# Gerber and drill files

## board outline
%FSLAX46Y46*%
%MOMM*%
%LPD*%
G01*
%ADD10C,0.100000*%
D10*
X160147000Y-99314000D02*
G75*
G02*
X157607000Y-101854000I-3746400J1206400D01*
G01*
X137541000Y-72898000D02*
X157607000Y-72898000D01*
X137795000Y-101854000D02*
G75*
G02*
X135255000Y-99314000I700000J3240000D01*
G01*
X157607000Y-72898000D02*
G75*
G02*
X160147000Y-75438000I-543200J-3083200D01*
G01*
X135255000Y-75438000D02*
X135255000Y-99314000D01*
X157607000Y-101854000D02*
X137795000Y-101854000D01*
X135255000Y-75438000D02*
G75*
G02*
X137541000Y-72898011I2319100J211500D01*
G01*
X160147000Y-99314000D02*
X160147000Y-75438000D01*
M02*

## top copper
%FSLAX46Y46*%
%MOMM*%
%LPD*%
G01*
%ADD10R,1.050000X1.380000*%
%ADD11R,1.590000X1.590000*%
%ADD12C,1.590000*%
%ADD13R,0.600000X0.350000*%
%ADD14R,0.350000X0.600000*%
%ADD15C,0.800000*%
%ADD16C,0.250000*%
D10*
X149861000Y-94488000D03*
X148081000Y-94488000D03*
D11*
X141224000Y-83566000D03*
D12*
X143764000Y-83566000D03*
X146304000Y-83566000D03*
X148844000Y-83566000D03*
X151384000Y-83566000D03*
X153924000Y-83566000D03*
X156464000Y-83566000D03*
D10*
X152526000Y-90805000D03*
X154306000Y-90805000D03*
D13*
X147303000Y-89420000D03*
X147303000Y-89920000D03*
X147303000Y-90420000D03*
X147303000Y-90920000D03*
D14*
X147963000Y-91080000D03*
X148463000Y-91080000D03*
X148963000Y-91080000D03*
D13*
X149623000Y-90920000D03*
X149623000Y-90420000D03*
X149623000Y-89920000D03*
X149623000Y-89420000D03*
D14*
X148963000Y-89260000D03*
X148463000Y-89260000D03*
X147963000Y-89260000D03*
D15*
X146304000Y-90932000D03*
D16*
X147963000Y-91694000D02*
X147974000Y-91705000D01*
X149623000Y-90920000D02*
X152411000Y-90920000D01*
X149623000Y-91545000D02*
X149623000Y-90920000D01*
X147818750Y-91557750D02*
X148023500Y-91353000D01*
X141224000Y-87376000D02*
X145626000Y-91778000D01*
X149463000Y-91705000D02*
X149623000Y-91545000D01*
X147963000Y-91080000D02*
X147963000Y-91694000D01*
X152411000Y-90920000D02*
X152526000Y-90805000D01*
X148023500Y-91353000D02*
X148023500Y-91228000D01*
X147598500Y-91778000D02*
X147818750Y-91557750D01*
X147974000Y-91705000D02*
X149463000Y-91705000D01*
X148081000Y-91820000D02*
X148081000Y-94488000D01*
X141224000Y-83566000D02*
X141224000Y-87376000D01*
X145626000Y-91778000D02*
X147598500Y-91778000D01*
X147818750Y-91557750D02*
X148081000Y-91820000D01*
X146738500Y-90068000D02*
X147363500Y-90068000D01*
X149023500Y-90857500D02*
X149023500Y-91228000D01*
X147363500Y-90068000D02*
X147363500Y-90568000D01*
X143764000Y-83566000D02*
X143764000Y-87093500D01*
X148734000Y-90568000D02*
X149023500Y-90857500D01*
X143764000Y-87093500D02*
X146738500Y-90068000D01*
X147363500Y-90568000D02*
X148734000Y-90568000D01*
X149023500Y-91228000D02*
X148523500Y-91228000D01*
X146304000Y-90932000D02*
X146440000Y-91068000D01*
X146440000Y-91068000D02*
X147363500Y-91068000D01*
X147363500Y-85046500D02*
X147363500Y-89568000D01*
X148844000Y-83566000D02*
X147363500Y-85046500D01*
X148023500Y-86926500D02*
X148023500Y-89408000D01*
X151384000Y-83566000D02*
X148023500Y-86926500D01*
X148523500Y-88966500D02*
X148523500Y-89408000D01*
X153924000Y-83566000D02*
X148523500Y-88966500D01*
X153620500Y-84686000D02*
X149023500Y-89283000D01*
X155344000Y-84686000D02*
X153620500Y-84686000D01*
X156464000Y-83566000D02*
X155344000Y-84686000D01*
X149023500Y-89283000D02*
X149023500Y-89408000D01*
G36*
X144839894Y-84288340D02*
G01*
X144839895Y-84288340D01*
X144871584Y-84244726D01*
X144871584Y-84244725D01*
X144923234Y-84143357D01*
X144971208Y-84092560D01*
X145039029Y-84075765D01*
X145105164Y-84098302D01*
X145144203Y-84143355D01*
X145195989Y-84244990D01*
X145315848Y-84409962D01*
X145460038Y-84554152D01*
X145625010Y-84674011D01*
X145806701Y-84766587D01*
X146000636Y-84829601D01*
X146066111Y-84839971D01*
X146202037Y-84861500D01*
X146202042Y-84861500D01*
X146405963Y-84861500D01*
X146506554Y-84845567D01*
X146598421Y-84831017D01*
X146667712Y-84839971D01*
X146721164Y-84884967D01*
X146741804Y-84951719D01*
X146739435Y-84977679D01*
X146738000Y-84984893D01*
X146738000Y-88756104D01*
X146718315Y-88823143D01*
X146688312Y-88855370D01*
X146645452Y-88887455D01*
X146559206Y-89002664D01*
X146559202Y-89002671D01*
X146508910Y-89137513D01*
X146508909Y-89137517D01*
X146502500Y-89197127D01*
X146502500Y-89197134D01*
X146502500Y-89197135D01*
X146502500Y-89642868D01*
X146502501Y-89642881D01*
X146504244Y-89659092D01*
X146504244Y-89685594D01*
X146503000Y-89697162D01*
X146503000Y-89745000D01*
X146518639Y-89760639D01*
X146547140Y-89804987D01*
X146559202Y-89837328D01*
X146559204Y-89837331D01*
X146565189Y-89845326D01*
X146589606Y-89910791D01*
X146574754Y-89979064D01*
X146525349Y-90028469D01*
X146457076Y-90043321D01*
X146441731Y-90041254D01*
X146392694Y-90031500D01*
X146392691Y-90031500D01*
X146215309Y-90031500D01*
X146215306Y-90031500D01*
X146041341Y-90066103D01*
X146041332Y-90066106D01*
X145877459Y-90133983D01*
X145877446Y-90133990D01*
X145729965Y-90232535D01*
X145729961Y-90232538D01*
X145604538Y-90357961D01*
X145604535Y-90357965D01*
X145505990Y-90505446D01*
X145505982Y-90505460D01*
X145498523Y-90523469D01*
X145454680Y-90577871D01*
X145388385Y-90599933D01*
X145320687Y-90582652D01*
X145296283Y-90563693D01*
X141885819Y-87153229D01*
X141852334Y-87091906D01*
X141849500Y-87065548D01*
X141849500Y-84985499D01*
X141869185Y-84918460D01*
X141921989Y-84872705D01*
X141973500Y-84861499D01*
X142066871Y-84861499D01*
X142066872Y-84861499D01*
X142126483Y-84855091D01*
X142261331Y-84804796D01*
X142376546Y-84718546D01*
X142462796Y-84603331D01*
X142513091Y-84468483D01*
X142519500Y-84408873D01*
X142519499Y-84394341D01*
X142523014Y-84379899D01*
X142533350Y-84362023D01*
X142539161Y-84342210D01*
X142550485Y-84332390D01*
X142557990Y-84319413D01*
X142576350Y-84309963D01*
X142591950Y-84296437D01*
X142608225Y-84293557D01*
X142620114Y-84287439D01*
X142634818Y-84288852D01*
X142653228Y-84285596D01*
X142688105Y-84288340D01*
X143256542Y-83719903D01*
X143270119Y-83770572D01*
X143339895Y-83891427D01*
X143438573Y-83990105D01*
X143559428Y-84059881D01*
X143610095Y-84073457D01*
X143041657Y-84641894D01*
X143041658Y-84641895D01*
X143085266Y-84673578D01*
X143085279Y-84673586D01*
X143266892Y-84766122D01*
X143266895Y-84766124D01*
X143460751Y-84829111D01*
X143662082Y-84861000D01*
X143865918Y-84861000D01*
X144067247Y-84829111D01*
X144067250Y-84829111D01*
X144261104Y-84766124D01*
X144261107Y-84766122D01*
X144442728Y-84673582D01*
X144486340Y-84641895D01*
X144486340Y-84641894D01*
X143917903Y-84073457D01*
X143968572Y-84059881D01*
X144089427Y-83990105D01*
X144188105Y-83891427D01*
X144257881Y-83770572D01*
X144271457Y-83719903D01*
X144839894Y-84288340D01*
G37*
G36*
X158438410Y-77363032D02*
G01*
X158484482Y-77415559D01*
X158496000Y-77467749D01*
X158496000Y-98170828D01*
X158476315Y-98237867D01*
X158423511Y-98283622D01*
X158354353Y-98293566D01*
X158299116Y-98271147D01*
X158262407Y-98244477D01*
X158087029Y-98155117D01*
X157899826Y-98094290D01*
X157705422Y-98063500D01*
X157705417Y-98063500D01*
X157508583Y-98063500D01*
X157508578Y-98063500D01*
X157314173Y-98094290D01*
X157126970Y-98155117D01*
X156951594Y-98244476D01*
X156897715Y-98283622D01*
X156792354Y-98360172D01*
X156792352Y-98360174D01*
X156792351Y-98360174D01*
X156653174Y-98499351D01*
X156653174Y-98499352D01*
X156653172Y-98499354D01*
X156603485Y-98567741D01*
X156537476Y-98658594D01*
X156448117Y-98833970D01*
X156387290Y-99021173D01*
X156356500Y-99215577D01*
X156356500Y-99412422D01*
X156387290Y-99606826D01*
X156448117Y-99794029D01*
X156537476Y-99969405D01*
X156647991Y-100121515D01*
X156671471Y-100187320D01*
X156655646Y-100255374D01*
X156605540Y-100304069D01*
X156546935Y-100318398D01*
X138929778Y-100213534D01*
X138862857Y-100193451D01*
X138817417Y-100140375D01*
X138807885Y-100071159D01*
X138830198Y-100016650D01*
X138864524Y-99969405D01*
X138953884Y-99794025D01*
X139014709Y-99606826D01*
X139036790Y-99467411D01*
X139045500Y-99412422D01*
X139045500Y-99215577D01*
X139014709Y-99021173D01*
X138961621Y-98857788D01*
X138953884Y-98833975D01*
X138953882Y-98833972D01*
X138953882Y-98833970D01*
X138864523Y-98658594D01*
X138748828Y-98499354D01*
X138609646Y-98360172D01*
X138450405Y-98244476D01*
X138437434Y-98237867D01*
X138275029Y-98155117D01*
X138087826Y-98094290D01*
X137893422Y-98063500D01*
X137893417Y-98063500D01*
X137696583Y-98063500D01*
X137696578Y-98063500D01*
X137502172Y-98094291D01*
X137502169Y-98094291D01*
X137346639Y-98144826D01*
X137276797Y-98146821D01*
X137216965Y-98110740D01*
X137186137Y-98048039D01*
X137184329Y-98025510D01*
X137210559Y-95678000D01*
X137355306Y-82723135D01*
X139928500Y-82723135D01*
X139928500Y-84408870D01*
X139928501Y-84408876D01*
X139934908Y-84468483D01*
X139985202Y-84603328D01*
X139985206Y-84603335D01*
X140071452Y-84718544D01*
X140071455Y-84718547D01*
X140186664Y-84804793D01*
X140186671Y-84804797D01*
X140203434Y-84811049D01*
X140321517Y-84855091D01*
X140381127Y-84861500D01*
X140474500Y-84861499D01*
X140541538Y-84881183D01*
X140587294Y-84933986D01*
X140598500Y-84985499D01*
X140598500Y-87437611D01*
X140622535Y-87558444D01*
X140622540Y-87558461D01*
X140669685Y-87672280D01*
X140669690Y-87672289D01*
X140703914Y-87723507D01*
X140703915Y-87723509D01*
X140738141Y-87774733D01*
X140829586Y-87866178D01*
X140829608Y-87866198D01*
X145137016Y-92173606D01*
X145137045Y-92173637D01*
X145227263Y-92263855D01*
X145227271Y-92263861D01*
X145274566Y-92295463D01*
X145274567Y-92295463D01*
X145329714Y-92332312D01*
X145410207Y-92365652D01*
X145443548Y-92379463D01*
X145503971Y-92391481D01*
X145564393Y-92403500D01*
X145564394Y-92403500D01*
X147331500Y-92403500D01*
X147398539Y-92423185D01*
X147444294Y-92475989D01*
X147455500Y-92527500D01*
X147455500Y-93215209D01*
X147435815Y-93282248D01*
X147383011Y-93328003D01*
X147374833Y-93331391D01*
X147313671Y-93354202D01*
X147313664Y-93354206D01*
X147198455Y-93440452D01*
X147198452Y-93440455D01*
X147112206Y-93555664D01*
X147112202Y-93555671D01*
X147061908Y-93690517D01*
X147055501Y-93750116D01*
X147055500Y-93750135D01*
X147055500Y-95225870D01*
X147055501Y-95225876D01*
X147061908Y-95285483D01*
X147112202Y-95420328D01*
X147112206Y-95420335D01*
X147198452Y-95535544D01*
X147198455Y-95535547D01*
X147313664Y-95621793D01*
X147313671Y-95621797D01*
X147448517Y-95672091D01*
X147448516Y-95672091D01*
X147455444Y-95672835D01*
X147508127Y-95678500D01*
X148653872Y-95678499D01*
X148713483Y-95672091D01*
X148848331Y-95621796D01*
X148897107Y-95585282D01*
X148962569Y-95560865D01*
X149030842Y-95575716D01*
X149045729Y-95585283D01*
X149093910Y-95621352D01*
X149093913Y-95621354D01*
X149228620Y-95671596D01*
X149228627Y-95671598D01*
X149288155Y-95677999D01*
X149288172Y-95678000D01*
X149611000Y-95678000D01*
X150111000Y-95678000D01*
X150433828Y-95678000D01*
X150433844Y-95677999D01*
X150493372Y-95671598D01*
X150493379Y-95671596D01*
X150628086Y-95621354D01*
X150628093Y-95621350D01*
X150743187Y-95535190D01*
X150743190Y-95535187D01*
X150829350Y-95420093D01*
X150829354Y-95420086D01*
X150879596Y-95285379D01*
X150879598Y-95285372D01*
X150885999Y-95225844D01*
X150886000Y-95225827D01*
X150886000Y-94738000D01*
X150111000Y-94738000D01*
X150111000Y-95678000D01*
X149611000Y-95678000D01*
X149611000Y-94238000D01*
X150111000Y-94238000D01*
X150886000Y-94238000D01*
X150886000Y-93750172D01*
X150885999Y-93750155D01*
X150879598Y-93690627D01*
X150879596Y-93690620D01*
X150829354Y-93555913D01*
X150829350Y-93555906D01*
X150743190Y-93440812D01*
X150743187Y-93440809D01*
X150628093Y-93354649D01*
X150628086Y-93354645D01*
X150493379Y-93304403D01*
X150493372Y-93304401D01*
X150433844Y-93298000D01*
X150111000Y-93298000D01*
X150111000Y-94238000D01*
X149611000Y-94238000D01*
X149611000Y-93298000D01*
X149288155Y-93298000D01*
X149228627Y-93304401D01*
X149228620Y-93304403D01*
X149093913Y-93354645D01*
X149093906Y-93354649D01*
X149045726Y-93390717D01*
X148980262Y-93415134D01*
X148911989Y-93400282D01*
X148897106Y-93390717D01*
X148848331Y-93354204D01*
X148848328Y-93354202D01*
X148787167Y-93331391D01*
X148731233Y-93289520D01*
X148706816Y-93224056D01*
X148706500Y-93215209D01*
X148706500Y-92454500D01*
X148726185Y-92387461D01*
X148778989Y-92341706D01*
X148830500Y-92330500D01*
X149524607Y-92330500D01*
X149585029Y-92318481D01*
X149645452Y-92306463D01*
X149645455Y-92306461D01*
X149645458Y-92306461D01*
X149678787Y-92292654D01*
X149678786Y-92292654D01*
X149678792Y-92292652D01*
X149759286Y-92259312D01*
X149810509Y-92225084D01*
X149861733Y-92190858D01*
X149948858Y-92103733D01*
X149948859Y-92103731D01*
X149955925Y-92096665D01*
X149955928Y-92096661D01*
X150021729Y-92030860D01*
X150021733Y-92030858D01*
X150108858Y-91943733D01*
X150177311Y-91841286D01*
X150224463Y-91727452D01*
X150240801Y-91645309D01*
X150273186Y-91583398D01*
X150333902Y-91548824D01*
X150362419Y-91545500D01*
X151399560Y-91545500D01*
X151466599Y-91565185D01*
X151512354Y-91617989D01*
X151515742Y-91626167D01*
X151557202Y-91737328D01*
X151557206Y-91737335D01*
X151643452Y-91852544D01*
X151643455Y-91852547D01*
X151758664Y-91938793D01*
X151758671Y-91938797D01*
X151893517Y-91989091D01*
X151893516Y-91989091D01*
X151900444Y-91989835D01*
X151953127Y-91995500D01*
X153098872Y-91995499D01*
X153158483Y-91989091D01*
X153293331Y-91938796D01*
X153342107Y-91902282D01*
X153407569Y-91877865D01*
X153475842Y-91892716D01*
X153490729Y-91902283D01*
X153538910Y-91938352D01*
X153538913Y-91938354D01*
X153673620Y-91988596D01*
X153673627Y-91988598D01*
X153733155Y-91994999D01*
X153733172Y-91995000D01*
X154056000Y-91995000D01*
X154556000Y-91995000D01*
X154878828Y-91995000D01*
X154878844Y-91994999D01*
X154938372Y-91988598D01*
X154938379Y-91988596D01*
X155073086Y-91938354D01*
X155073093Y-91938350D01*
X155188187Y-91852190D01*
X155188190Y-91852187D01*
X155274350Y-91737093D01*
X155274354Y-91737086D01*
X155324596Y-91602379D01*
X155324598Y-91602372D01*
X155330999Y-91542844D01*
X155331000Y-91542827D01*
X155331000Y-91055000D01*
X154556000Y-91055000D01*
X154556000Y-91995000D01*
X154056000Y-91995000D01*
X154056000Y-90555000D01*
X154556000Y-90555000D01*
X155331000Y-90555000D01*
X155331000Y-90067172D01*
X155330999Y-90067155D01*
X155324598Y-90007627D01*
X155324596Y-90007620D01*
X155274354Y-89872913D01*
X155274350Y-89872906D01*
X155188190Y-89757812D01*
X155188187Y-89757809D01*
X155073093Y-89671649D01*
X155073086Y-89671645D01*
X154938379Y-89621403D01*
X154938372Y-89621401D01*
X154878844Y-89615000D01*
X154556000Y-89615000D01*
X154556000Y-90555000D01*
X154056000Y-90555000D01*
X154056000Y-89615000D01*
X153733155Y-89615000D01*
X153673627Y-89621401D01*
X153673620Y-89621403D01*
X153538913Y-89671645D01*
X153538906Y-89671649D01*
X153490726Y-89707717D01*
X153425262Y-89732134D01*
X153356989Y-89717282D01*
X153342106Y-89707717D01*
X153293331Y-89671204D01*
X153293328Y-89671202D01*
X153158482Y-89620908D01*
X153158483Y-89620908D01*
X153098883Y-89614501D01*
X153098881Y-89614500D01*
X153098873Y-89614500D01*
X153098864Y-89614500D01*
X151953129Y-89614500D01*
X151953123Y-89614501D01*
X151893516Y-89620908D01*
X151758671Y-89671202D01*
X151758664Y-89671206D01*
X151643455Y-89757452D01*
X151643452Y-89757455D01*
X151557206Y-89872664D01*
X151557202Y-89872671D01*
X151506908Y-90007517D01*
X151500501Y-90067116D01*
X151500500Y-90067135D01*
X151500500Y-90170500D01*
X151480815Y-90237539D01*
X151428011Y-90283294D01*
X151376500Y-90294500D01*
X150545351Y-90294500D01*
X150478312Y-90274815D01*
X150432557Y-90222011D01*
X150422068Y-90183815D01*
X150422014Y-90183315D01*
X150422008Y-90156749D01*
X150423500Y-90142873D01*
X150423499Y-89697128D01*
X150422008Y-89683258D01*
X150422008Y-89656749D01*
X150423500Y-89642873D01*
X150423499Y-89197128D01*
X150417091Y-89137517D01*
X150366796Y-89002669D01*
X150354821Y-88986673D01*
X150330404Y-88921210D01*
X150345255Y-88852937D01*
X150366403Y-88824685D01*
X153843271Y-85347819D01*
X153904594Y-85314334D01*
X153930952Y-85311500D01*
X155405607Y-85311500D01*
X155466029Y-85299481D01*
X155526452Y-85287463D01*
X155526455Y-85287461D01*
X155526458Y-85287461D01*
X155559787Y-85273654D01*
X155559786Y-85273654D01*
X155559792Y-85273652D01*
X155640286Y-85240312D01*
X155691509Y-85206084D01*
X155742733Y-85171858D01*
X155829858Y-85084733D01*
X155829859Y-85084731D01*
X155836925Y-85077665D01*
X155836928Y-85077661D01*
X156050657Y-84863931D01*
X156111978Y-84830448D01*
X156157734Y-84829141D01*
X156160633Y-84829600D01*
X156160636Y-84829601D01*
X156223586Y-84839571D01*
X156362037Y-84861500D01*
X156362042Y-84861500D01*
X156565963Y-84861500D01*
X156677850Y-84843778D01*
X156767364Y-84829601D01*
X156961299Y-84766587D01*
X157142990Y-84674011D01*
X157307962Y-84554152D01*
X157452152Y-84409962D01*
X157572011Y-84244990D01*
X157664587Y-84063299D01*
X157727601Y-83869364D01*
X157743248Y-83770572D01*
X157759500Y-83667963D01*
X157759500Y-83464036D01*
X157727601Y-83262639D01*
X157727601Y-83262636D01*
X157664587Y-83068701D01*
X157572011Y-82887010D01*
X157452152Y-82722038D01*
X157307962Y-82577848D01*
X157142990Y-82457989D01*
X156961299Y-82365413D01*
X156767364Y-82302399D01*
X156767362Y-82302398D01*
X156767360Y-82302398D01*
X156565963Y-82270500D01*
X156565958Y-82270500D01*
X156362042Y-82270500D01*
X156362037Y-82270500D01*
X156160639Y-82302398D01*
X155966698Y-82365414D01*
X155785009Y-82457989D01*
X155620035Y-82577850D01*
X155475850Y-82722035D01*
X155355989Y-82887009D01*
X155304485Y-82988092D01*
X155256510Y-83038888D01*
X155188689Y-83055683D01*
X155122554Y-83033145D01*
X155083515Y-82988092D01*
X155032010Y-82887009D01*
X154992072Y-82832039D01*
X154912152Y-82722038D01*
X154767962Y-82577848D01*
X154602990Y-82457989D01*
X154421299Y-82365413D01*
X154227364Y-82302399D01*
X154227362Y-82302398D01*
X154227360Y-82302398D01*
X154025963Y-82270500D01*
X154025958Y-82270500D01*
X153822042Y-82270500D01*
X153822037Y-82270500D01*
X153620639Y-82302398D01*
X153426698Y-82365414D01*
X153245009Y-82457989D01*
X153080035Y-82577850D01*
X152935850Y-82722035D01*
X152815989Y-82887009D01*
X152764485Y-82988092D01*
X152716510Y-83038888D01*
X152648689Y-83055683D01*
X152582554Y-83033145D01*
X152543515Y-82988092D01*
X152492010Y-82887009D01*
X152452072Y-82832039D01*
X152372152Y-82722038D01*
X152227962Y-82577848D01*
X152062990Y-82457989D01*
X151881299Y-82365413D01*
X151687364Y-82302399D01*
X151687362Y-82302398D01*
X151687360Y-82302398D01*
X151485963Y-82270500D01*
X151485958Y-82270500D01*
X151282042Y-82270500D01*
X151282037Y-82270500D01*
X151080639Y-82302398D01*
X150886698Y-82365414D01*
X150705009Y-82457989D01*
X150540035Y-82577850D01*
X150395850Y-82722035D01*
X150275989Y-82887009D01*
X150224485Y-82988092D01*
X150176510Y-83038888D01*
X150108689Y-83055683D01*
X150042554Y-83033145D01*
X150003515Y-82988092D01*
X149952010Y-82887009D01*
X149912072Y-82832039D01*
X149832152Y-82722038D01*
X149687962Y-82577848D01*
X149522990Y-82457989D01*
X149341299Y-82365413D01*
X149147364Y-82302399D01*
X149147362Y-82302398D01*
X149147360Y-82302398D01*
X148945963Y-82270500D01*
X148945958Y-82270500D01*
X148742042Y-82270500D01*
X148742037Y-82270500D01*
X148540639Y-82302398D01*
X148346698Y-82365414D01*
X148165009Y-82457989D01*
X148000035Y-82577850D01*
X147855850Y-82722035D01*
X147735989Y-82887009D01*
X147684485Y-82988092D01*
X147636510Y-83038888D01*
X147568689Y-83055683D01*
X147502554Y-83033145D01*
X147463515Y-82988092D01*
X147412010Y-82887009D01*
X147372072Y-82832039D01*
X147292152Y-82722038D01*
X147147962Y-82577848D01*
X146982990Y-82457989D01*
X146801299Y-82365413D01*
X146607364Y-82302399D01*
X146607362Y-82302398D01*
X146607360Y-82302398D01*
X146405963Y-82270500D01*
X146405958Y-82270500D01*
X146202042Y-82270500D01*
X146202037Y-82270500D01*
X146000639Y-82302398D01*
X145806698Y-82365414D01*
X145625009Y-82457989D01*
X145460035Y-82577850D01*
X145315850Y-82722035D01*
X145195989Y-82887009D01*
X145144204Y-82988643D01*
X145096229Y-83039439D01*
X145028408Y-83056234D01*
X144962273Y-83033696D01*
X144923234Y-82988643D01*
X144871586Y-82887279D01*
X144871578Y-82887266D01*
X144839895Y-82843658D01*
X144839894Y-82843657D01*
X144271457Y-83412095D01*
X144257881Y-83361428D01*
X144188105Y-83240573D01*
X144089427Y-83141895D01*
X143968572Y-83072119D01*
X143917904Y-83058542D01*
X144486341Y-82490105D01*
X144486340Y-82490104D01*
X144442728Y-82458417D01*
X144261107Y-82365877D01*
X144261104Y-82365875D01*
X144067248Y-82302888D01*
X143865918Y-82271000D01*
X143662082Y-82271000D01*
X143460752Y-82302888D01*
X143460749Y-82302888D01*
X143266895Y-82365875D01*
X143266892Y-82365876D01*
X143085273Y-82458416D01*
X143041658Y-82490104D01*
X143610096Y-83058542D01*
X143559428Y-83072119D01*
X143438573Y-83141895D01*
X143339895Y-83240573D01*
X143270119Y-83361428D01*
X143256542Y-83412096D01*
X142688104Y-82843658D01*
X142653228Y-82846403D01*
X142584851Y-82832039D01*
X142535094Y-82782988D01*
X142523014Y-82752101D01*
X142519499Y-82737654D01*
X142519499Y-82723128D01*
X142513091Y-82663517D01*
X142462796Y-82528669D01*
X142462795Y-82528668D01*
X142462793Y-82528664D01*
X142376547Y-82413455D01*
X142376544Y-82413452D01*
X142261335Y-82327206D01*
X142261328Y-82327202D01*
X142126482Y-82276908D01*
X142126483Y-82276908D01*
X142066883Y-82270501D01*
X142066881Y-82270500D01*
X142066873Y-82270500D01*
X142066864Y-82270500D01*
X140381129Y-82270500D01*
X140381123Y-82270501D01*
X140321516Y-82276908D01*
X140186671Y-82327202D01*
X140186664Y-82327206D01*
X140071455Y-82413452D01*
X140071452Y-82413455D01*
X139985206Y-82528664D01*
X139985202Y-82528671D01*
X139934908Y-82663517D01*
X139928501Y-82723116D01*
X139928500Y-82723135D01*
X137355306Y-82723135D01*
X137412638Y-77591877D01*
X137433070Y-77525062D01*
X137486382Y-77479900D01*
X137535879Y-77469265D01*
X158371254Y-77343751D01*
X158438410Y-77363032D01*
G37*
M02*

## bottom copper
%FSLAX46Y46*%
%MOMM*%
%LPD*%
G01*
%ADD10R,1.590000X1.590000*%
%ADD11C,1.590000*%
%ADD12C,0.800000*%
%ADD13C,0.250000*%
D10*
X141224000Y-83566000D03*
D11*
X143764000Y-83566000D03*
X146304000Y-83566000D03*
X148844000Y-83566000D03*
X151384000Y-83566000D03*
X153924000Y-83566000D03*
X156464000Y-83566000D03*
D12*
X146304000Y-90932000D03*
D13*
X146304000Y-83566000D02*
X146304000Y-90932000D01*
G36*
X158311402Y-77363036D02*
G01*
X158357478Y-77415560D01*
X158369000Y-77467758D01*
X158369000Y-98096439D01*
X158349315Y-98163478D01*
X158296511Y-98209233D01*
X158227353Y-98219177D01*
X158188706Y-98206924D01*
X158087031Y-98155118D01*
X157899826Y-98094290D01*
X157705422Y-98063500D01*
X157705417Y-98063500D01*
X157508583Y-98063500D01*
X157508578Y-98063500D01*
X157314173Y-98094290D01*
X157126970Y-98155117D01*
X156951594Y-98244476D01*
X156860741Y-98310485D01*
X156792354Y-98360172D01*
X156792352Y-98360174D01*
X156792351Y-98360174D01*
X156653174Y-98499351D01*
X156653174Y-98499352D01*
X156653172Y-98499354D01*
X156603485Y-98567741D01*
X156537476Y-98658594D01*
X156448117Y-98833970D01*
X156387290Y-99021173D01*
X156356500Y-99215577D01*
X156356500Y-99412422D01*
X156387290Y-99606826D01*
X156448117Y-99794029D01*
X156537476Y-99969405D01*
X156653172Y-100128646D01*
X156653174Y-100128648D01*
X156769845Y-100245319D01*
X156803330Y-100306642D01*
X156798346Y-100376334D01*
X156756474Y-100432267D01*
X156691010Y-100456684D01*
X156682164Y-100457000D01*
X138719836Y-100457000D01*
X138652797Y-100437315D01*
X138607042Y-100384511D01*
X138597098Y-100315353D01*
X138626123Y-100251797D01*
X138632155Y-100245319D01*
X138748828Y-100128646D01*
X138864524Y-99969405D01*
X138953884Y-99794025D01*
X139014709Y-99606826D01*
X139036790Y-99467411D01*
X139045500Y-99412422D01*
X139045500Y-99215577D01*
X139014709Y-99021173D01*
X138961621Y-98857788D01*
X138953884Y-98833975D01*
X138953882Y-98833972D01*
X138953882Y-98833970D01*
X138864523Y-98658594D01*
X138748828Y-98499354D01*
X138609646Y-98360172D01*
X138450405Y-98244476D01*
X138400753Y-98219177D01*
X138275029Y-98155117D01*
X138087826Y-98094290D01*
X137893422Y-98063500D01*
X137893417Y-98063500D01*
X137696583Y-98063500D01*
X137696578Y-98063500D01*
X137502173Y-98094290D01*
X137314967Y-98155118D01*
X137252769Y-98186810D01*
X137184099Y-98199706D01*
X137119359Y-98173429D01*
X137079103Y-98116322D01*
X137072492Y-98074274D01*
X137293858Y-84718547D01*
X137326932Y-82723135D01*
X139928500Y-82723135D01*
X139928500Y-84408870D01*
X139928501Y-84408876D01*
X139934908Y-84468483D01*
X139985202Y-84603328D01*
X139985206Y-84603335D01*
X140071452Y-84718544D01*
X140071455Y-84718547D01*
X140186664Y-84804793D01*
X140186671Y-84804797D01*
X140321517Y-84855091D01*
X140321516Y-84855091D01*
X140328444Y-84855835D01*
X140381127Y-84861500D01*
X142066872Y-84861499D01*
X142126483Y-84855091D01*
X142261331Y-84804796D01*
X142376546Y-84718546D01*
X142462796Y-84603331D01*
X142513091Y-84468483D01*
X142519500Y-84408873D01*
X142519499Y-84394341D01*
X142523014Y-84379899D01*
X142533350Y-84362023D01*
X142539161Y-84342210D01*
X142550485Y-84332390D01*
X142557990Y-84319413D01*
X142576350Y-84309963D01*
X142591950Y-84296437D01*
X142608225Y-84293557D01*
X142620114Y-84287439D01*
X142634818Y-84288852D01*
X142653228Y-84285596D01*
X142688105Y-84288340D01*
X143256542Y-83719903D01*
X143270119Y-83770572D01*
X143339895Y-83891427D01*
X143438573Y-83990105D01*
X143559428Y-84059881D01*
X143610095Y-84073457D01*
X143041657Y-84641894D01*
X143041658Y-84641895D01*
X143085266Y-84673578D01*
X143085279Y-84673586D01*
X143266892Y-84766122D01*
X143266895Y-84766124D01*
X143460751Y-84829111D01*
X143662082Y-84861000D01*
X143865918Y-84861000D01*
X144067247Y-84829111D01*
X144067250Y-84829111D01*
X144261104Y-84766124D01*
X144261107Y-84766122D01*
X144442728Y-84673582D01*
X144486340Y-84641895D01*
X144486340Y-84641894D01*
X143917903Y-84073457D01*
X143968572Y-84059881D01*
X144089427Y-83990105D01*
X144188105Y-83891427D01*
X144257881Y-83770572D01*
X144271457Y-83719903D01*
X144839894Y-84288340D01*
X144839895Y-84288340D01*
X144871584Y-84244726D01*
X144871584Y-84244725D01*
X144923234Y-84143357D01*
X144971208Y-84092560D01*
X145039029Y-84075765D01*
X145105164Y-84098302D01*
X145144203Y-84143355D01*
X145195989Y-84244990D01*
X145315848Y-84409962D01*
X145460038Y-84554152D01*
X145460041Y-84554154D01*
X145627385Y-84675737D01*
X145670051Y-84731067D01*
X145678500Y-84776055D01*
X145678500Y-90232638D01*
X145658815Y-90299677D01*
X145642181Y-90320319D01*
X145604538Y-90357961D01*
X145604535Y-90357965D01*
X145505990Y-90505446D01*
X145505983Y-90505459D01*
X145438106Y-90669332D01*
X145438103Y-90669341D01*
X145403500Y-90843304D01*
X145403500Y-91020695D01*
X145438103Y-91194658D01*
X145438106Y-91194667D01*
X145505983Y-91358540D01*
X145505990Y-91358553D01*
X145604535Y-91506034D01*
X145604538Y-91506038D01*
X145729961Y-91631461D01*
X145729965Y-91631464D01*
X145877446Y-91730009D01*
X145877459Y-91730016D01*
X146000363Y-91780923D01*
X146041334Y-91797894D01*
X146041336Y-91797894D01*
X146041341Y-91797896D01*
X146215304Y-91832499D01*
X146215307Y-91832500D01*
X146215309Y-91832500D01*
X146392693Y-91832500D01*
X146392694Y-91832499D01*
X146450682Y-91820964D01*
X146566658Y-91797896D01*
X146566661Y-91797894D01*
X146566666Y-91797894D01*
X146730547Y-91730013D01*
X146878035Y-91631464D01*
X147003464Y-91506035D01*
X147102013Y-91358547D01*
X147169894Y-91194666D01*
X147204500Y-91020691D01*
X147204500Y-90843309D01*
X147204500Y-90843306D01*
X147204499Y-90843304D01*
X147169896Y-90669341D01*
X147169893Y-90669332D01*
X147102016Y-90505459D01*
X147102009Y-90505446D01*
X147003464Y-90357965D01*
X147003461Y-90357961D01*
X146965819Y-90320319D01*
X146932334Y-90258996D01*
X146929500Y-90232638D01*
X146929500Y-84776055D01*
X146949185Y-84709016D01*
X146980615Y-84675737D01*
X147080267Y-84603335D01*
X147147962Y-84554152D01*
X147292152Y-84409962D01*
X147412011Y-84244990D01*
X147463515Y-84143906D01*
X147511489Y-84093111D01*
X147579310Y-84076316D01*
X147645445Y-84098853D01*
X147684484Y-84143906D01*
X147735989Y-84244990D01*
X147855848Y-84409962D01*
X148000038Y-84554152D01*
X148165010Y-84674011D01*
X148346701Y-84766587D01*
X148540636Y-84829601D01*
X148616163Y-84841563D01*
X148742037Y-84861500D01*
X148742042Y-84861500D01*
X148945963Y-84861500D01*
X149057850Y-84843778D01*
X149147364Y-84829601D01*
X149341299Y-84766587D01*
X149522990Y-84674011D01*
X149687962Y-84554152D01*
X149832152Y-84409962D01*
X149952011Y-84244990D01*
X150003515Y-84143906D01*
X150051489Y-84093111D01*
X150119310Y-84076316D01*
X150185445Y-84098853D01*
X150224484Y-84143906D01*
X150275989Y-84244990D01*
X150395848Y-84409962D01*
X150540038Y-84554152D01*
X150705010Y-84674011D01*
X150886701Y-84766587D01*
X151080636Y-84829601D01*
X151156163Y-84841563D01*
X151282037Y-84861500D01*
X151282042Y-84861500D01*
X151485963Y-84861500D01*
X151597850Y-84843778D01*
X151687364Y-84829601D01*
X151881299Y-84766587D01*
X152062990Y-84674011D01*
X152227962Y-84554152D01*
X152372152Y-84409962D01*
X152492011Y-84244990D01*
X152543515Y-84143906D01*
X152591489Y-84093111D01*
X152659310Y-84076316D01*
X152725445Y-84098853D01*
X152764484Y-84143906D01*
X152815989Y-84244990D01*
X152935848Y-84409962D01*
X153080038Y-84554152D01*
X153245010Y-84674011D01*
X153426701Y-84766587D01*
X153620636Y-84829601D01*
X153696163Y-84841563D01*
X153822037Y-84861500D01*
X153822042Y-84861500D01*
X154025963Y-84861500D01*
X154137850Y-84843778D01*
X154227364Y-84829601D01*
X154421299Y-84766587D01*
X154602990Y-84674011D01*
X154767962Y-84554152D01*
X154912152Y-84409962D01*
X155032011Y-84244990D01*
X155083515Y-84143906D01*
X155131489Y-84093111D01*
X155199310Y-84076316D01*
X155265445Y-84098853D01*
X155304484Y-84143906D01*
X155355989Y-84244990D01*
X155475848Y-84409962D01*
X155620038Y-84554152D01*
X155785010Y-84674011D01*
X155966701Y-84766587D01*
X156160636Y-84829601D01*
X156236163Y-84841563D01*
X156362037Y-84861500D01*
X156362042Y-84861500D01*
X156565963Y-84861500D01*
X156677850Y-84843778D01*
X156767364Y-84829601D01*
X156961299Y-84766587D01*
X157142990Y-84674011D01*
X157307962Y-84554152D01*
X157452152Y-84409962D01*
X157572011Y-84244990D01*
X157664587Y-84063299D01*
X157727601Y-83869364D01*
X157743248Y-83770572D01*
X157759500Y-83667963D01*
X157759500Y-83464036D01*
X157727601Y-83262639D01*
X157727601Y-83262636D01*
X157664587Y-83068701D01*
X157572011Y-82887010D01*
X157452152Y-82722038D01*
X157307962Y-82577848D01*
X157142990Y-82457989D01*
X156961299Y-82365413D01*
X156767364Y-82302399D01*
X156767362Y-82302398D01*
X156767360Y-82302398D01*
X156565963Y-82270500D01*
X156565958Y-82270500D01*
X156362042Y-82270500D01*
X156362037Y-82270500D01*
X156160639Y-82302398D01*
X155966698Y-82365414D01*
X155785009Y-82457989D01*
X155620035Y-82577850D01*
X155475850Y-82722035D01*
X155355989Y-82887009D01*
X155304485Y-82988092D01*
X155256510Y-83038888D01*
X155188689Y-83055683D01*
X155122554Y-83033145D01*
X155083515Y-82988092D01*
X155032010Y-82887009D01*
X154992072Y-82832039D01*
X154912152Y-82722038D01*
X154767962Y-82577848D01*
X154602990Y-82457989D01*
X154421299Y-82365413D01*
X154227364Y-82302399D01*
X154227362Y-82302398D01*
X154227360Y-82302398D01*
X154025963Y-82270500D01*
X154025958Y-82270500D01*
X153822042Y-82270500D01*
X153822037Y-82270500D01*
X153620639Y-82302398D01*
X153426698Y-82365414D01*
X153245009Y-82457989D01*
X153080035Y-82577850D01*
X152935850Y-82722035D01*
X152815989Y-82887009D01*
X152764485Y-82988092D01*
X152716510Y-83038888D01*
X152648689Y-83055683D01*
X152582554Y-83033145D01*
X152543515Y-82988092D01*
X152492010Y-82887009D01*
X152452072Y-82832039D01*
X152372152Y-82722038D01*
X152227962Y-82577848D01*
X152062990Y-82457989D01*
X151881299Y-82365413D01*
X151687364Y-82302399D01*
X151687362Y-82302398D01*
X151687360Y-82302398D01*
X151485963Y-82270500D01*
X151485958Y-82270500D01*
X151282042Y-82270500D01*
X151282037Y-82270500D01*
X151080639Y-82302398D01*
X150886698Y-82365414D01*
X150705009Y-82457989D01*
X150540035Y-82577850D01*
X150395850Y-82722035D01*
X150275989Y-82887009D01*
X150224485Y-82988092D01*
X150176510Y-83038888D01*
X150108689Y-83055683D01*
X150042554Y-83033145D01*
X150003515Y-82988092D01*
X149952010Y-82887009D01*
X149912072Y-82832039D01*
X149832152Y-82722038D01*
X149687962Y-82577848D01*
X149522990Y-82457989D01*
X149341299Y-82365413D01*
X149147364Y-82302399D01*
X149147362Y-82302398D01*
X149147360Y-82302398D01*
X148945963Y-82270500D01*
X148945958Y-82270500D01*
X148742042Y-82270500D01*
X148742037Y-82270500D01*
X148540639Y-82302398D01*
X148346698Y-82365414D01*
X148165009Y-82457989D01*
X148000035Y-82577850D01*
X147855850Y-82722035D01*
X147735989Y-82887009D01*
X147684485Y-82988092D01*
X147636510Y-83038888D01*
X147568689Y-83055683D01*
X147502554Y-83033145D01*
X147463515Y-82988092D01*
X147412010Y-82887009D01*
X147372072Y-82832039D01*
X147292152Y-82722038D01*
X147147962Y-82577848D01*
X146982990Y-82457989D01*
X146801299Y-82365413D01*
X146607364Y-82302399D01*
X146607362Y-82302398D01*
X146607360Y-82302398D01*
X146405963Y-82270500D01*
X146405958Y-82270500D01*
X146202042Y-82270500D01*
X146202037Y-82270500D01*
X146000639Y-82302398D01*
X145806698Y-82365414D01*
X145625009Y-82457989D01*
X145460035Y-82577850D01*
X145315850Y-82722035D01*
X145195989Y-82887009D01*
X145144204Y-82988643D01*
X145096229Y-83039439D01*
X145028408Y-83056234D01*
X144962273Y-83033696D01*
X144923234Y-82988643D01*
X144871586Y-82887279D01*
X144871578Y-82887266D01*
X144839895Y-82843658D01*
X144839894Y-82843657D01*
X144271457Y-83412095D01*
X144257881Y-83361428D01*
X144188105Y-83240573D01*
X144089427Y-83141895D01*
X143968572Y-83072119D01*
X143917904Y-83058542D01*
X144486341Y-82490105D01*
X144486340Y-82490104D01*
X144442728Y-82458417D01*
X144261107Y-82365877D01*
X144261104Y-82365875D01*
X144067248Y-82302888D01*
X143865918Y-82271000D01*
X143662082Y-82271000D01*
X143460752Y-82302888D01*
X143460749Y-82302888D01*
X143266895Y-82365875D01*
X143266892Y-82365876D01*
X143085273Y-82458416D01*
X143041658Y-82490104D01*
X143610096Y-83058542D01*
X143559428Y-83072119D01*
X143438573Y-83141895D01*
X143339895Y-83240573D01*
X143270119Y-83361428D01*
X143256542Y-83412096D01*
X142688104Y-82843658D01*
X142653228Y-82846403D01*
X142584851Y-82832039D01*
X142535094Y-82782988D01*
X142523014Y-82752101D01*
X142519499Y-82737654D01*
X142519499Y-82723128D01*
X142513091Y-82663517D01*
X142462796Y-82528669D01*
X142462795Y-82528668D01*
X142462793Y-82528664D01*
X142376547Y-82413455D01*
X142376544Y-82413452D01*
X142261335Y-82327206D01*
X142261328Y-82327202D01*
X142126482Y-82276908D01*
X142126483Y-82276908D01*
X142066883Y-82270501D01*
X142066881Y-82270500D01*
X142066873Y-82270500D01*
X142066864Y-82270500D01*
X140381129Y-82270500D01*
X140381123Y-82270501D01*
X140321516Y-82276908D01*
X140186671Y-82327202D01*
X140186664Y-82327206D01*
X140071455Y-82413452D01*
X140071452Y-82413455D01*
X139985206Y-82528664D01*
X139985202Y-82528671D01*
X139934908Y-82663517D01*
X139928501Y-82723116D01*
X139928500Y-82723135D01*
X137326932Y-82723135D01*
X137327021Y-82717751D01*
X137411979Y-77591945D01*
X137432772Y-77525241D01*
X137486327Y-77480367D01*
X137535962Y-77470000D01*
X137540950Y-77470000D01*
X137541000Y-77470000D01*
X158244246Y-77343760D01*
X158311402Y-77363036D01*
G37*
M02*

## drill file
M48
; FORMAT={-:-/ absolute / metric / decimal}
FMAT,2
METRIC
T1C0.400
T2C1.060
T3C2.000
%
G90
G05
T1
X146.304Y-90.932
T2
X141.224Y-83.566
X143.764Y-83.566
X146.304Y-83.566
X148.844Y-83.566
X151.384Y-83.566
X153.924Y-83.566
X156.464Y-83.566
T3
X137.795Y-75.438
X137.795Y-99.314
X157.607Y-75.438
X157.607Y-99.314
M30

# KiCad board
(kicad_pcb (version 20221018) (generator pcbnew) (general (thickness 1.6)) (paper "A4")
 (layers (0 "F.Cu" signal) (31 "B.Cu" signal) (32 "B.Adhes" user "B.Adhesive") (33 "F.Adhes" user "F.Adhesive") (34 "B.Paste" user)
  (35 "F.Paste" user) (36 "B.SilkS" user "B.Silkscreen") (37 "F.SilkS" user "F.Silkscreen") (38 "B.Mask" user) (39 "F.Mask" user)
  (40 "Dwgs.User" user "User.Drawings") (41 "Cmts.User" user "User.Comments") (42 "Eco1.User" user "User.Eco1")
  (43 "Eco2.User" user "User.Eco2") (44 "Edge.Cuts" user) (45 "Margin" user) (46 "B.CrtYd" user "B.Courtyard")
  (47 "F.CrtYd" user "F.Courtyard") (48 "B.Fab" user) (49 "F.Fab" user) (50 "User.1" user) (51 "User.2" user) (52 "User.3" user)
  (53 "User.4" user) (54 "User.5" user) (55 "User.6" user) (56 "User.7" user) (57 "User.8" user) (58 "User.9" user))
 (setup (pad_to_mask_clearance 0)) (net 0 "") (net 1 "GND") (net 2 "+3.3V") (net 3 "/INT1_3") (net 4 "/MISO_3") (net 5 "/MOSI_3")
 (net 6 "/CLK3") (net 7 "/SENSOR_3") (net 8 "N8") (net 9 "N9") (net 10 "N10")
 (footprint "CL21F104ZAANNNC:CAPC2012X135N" (layer "F.Cu") (at 148.971 94.488 180)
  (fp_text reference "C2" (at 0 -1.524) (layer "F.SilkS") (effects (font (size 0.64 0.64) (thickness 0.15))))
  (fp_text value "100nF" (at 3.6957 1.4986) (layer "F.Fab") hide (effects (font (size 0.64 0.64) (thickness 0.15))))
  (pad "1" smd rect (at -0.89 0 180) (size 1.05 1.38) (layers "F.Cu" "F.Paste" "F.Mask") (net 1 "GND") (solder_mask_margin 0.102))
  (pad "2" smd rect (at 0.89 0 180) (size 1.05 1.38) (layers "F.Cu" "F.Paste" "F.Mask") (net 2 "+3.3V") (solder_mask_margin 0.102)))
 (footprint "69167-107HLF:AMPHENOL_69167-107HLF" (layer "F.Cu") (at 148.844 83.566)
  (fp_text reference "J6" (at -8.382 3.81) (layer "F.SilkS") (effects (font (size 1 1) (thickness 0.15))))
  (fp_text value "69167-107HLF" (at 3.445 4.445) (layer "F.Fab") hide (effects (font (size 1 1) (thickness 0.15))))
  (pad "01" thru_hole rect (at -7.62 0) (size 1.59 1.59) (drill 1.06) (layers "*.Cu" "*.Mask") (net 2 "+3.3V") (solder_mask_margin 0.102))
  (pad "02" thru_hole circle (at -5.08 0) (size 1.59 1.59) (drill 1.06) (layers "*.Cu" "*.Mask") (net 1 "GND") (solder_mask_margin 0.102))
  (pad "03" thru_hole circle (at -2.54 0) (size 1.59 1.59) (drill 1.06) (layers "*.Cu" "*.Mask") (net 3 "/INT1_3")
   (solder_mask_margin 0.102))
  (pad "04" thru_hole circle (at 0 0) (size 1.59 1.59) (drill 1.06) (layers "*.Cu" "*.Mask") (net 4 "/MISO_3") (solder_mask_margin 0.102))
  (pad "05" thru_hole circle (at 2.54 0) (size 1.59 1.59) (drill 1.06) (layers "*.Cu" "*.Mask") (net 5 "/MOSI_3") (solder_mask_margin 0.102))
  (pad "06" thru_hole circle (at 5.08 0) (size 1.59 1.59) (drill 1.06) (layers "*.Cu" "*.Mask") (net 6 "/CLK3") (solder_mask_margin 0.102))
  (pad "07" thru_hole circle (at 7.62 0) (size 1.59 1.59) (drill 1.06) (layers "*.Cu" "*.Mask") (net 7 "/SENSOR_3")
   (solder_mask_margin 0.102)))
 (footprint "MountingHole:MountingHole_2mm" (layer "F.Cu") (at 137.795 75.438)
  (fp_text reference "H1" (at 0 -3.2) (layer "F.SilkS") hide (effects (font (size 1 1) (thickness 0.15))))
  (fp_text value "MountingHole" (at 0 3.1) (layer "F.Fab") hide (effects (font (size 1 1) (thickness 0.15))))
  (pad "" np_thru_hole circle (at 0 0) (size 2 2) (drill 2) (layers "*.Cu" "*.Mask")))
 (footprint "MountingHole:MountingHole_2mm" (layer "F.Cu") (at 157.607 75.438)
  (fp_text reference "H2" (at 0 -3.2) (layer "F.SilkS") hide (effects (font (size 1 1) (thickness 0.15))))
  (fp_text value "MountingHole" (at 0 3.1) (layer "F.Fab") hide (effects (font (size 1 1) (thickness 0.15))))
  (pad "" np_thru_hole circle (at 0 0) (size 2 2) (drill 2) (layers "*.Cu" "*.Mask")))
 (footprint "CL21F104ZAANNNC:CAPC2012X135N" (layer "F.Cu") (at 153.416 90.805)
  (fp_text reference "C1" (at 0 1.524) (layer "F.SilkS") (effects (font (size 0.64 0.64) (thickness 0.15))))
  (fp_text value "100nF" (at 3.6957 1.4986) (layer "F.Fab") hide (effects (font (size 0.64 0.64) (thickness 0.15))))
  (pad "1" smd rect (at -0.89 0) (size 1.05 1.38) (layers "F.Cu" "F.Paste" "F.Mask") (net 2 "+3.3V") (solder_mask_margin 0.102))
  (pad "2" smd rect (at 0.89 0) (size 1.05 1.38) (layers "F.Cu" "F.Paste" "F.Mask") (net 1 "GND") (solder_mask_margin 0.102)))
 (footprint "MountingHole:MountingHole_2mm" (layer "F.Cu") (at 157.607 99.314)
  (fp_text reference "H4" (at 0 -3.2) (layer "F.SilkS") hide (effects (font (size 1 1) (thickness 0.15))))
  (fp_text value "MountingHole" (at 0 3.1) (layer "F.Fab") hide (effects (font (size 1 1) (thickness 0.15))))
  (pad "" np_thru_hole circle (at 0 0) (size 2 2) (drill 2) (layers "*.Cu" "*.Mask")))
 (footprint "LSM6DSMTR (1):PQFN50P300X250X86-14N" (layer "F.Cu") (at 148.463 90.17)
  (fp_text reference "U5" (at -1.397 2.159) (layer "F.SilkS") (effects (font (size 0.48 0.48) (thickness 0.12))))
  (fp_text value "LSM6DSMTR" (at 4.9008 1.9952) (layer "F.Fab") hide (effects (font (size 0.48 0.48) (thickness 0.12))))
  (pad "1" smd rect (at -1.16 -0.75) (size 0.6 0.35) (layers "F.Cu" "F.Paste" "F.Mask") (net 4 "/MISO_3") (solder_mask_margin 0.102))
  (pad "2" smd rect (at -1.16 -0.25) (size 0.6 0.35) (layers "F.Cu" "F.Paste" "F.Mask") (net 1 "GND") (solder_mask_margin 0.102))
  (pad "3" smd rect (at -1.16 0.25) (size 0.6 0.35) (layers "F.Cu" "F.Paste" "F.Mask") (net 1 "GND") (solder_mask_margin 0.102))
  (pad "4" smd rect (at -1.16 0.75) (size 0.6 0.35) (layers "F.Cu" "F.Paste" "F.Mask") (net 3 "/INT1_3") (solder_mask_margin 0.102))
  (pad "5" smd rect (at -0.5 0.91 90) (size 0.6 0.35) (layers "F.Cu" "F.Paste" "F.Mask") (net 2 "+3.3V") (solder_mask_margin 0.102))
  (pad "6" smd rect (at 0 0.91 90) (size 0.6 0.35) (layers "F.Cu" "F.Paste" "F.Mask") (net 1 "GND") (solder_mask_margin 0.102))
  (pad "7" smd rect (at 0.5 0.91 90) (size 0.6 0.35) (layers "F.Cu" "F.Paste" "F.Mask") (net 1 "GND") (solder_mask_margin 0.102))
  (pad "8" smd rect (at 1.16 0.75) (size 0.6 0.35) (layers "F.Cu" "F.Paste" "F.Mask") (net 2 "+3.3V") (solder_mask_margin 0.102))
  (pad "9" smd rect (at 1.16 0.25) (size 0.6 0.35) (layers "F.Cu" "F.Paste" "F.Mask") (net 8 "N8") (solder_mask_margin 0.102))
  (pad "10" smd rect (at 1.16 -0.25) (size 0.6 0.35) (layers "F.Cu" "F.Paste" "F.Mask") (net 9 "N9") (solder_mask_margin 0.102))
  (pad "11" smd rect (at 1.16 -0.75) (size 0.6 0.35) (layers "F.Cu" "F.Paste" "F.Mask") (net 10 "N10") (solder_mask_margin 0.102))
  (pad "12" smd rect (at 0.5 -0.91 90) (size 0.6 0.35) (layers "F.Cu" "F.Paste" "F.Mask") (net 7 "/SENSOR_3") (solder_mask_margin 0.102))
  (pad "13" smd rect (at 0 -0.91 90) (size 0.6 0.35) (layers "F.Cu" "F.Paste" "F.Mask") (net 6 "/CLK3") (solder_mask_margin 0.102))
  (pad "14" smd rect (at -0.5 -0.91 90) (size 0.6 0.35) (layers "F.Cu" "F.Paste" "F.Mask") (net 5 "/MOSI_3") (solder_mask_margin 0.102)))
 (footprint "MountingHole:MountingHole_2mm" (layer "F.Cu") (at 137.795 99.314)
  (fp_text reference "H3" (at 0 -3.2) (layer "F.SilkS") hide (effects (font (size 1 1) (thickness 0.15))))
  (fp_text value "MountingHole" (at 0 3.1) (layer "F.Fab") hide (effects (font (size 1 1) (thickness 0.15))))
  (pad "" np_thru_hole circle (at 0 0) (size 2 2) (drill 2) (layers "*.Cu" "*.Mask")))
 (gr_arc (start 160.147 99.314) (mid 159.183666 100.890666) (end 157.607 101.854) (stroke (width 0.1) (type default)) (layer "Edge.Cuts"))
 (gr_line (start 137.541 72.898) (end 157.607 72.898) (stroke (width 0.1) (type default)) (layer "Edge.Cuts"))
 (gr_arc (start 137.795 101.854) (mid 136.151114 100.957886) (end 135.255 99.314) (stroke (width 0.1) (type default)) (layer "Edge.Cuts"))
 (gr_arc (start 157.607 72.898) (mid 159.277529 73.767471) (end 160.147 75.438) (stroke (width 0.1) (type default)) (layer "Edge.Cuts"))
 (gr_line (start 135.255 75.438) (end 135.255 99.314) (stroke (width 0.1) (type default)) (layer "Edge.Cuts"))
 (gr_line (start 157.607 101.854) (end 137.795 101.854) (stroke (width 0.1) (type default)) (layer "Edge.Cuts"))
 (gr_arc (start 135.255 75.438) (mid 135.843178 73.66866) (end 137.541 72.898) (stroke (width 0.1) (type default)) (layer "Edge.Cuts"))
 (gr_line (start 160.147 99.314) (end 160.147 75.438) (stroke (width 0.1) (type default)) (layer "Edge.Cuts"))
 (segment (start 147.963 91.694) (end 147.974 91.705) (width 0.25) (layer "F.Cu") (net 2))
 (segment (start 149.623 90.92) (end 152.411 90.92) (width 0.25) (layer "F.Cu") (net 2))
 (segment (start 149.623 91.545) (end 149.623 90.92) (width 0.25) (layer "F.Cu") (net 2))
 (segment (start 147.81875 91.55775) (end 148.0235 91.353) (width 0.25) (layer "F.Cu") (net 2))
 (segment (start 141.224 87.376) (end 145.626 91.778) (width 0.25) (layer "F.Cu") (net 2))
 (segment (start 149.463 91.705) (end 149.623 91.545) (width 0.25) (layer "F.Cu") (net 2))
 (segment (start 147.963 91.08) (end 147.963 91.694) (width 0.25) (layer "F.Cu") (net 2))
 (segment (start 152.411 90.92) (end 152.526 90.805) (width 0.25) (layer "F.Cu") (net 2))
 (segment (start 148.0235 91.353) (end 148.0235 91.228) (width 0.25) (layer "F.Cu") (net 2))
 (segment (start 147.5985 91.778) (end 147.81875 91.55775) (width 0.25) (layer "F.Cu") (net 2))
 (segment (start 147.974 91.705) (end 149.463 91.705) (width 0.25) (layer "F.Cu") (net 2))
 (segment (start 148.081 91.82) (end 148.081 94.488) (width 0.25) (layer "F.Cu") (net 2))
 (segment (start 141.224 83.566) (end 141.224 87.376) (width 0.25) (layer "F.Cu") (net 2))
 (segment (start 145.626 91.778) (end 147.5985 91.778) (width 0.25) (layer "F.Cu") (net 2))
 (segment (start 147.81875 91.55775) (end 148.081 91.82) (width 0.25) (layer "F.Cu") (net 2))
 (segment (start 146.7385 90.068) (end 147.3635 90.068) (width 0.25) (layer "F.Cu") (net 1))
 (segment (start 149.0235 90.8575) (end 149.0235 91.228) (width 0.25) (layer "F.Cu") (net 1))
 (segment (start 147.3635 90.068) (end 147.3635 90.568) (width 0.25) (layer "F.Cu") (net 1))
 (segment (start 143.764 83.566) (end 143.764 87.0935) (width 0.25) (layer "F.Cu") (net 1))
 (segment (start 148.734 90.568) (end 149.0235 90.8575) (width 0.25) (layer "F.Cu") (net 1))
 (segment (start 143.764 87.0935) (end 146.7385 90.068) (width 0.25) (layer "F.Cu") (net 1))
 (segment (start 147.3635 90.568) (end 148.734 90.568) (width 0.25) (layer "F.Cu") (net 1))
 (segment (start 149.0235 91.228) (end 148.5235 91.228) (width 0.25) (layer "F.Cu") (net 1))
 (segment (start 146.304 90.932) (end 146.44 91.068) (width 0.25) (layer "F.Cu") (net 3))
 (segment (start 146.44 91.068) (end 147.3635 91.068) (width 0.25) (layer "F.Cu") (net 3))
 (via (at 146.304 90.932) (size 0.8) (drill 0.4) (layers "F.Cu" "B.Cu") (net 3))
 (segment (start 146.304 83.566) (end 146.304 90.932) (width 0.25) (layer "B.Cu") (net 3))
 (segment (start 147.3635 85.0465) (end 147.3635 89.568) (width 0.25) (layer "F.Cu") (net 4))
 (segment (start 148.844 83.566) (end 147.3635 85.0465) (width 0.25) (layer "F.Cu") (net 4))
 (segment (start 148.0235 86.9265) (end 148.0235 89.408) (width 0.25) (layer "F.Cu") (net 5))
 (segment (start 151.384 83.566) (end 148.0235 86.9265) (width 0.25) (layer "F.Cu") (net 5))
 (segment (start 148.5235 88.9665) (end 148.5235 89.408) (width 0.25) (layer "F.Cu") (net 6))
 (segment (start 153.924 83.566) (end 148.5235 88.9665) (width 0.25) (layer "F.Cu") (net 6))
 (segment (start 153.6205 84.686) (end 149.0235 89.283) (width 0.25) (layer "F.Cu") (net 7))
 (segment (start 155.344 84.686) (end 153.6205 84.686) (width 0.25) (layer "F.Cu") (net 7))
 (segment (start 156.464 83.566) (end 155.344 84.686) (width 0.25) (layer "F.Cu") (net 7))
 (segment (start 149.0235 89.283) (end 149.0235 89.408) (width 0.25) (layer "F.Cu") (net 7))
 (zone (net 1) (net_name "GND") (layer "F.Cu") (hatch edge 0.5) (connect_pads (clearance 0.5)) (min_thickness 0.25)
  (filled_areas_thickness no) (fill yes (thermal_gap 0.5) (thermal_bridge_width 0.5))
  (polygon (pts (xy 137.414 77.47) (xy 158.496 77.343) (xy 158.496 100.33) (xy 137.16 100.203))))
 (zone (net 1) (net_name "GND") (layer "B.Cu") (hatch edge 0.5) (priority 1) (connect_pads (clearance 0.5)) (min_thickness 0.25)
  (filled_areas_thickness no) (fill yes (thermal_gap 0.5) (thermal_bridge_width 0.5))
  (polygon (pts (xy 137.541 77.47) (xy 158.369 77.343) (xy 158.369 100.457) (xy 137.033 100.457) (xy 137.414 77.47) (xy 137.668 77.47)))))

